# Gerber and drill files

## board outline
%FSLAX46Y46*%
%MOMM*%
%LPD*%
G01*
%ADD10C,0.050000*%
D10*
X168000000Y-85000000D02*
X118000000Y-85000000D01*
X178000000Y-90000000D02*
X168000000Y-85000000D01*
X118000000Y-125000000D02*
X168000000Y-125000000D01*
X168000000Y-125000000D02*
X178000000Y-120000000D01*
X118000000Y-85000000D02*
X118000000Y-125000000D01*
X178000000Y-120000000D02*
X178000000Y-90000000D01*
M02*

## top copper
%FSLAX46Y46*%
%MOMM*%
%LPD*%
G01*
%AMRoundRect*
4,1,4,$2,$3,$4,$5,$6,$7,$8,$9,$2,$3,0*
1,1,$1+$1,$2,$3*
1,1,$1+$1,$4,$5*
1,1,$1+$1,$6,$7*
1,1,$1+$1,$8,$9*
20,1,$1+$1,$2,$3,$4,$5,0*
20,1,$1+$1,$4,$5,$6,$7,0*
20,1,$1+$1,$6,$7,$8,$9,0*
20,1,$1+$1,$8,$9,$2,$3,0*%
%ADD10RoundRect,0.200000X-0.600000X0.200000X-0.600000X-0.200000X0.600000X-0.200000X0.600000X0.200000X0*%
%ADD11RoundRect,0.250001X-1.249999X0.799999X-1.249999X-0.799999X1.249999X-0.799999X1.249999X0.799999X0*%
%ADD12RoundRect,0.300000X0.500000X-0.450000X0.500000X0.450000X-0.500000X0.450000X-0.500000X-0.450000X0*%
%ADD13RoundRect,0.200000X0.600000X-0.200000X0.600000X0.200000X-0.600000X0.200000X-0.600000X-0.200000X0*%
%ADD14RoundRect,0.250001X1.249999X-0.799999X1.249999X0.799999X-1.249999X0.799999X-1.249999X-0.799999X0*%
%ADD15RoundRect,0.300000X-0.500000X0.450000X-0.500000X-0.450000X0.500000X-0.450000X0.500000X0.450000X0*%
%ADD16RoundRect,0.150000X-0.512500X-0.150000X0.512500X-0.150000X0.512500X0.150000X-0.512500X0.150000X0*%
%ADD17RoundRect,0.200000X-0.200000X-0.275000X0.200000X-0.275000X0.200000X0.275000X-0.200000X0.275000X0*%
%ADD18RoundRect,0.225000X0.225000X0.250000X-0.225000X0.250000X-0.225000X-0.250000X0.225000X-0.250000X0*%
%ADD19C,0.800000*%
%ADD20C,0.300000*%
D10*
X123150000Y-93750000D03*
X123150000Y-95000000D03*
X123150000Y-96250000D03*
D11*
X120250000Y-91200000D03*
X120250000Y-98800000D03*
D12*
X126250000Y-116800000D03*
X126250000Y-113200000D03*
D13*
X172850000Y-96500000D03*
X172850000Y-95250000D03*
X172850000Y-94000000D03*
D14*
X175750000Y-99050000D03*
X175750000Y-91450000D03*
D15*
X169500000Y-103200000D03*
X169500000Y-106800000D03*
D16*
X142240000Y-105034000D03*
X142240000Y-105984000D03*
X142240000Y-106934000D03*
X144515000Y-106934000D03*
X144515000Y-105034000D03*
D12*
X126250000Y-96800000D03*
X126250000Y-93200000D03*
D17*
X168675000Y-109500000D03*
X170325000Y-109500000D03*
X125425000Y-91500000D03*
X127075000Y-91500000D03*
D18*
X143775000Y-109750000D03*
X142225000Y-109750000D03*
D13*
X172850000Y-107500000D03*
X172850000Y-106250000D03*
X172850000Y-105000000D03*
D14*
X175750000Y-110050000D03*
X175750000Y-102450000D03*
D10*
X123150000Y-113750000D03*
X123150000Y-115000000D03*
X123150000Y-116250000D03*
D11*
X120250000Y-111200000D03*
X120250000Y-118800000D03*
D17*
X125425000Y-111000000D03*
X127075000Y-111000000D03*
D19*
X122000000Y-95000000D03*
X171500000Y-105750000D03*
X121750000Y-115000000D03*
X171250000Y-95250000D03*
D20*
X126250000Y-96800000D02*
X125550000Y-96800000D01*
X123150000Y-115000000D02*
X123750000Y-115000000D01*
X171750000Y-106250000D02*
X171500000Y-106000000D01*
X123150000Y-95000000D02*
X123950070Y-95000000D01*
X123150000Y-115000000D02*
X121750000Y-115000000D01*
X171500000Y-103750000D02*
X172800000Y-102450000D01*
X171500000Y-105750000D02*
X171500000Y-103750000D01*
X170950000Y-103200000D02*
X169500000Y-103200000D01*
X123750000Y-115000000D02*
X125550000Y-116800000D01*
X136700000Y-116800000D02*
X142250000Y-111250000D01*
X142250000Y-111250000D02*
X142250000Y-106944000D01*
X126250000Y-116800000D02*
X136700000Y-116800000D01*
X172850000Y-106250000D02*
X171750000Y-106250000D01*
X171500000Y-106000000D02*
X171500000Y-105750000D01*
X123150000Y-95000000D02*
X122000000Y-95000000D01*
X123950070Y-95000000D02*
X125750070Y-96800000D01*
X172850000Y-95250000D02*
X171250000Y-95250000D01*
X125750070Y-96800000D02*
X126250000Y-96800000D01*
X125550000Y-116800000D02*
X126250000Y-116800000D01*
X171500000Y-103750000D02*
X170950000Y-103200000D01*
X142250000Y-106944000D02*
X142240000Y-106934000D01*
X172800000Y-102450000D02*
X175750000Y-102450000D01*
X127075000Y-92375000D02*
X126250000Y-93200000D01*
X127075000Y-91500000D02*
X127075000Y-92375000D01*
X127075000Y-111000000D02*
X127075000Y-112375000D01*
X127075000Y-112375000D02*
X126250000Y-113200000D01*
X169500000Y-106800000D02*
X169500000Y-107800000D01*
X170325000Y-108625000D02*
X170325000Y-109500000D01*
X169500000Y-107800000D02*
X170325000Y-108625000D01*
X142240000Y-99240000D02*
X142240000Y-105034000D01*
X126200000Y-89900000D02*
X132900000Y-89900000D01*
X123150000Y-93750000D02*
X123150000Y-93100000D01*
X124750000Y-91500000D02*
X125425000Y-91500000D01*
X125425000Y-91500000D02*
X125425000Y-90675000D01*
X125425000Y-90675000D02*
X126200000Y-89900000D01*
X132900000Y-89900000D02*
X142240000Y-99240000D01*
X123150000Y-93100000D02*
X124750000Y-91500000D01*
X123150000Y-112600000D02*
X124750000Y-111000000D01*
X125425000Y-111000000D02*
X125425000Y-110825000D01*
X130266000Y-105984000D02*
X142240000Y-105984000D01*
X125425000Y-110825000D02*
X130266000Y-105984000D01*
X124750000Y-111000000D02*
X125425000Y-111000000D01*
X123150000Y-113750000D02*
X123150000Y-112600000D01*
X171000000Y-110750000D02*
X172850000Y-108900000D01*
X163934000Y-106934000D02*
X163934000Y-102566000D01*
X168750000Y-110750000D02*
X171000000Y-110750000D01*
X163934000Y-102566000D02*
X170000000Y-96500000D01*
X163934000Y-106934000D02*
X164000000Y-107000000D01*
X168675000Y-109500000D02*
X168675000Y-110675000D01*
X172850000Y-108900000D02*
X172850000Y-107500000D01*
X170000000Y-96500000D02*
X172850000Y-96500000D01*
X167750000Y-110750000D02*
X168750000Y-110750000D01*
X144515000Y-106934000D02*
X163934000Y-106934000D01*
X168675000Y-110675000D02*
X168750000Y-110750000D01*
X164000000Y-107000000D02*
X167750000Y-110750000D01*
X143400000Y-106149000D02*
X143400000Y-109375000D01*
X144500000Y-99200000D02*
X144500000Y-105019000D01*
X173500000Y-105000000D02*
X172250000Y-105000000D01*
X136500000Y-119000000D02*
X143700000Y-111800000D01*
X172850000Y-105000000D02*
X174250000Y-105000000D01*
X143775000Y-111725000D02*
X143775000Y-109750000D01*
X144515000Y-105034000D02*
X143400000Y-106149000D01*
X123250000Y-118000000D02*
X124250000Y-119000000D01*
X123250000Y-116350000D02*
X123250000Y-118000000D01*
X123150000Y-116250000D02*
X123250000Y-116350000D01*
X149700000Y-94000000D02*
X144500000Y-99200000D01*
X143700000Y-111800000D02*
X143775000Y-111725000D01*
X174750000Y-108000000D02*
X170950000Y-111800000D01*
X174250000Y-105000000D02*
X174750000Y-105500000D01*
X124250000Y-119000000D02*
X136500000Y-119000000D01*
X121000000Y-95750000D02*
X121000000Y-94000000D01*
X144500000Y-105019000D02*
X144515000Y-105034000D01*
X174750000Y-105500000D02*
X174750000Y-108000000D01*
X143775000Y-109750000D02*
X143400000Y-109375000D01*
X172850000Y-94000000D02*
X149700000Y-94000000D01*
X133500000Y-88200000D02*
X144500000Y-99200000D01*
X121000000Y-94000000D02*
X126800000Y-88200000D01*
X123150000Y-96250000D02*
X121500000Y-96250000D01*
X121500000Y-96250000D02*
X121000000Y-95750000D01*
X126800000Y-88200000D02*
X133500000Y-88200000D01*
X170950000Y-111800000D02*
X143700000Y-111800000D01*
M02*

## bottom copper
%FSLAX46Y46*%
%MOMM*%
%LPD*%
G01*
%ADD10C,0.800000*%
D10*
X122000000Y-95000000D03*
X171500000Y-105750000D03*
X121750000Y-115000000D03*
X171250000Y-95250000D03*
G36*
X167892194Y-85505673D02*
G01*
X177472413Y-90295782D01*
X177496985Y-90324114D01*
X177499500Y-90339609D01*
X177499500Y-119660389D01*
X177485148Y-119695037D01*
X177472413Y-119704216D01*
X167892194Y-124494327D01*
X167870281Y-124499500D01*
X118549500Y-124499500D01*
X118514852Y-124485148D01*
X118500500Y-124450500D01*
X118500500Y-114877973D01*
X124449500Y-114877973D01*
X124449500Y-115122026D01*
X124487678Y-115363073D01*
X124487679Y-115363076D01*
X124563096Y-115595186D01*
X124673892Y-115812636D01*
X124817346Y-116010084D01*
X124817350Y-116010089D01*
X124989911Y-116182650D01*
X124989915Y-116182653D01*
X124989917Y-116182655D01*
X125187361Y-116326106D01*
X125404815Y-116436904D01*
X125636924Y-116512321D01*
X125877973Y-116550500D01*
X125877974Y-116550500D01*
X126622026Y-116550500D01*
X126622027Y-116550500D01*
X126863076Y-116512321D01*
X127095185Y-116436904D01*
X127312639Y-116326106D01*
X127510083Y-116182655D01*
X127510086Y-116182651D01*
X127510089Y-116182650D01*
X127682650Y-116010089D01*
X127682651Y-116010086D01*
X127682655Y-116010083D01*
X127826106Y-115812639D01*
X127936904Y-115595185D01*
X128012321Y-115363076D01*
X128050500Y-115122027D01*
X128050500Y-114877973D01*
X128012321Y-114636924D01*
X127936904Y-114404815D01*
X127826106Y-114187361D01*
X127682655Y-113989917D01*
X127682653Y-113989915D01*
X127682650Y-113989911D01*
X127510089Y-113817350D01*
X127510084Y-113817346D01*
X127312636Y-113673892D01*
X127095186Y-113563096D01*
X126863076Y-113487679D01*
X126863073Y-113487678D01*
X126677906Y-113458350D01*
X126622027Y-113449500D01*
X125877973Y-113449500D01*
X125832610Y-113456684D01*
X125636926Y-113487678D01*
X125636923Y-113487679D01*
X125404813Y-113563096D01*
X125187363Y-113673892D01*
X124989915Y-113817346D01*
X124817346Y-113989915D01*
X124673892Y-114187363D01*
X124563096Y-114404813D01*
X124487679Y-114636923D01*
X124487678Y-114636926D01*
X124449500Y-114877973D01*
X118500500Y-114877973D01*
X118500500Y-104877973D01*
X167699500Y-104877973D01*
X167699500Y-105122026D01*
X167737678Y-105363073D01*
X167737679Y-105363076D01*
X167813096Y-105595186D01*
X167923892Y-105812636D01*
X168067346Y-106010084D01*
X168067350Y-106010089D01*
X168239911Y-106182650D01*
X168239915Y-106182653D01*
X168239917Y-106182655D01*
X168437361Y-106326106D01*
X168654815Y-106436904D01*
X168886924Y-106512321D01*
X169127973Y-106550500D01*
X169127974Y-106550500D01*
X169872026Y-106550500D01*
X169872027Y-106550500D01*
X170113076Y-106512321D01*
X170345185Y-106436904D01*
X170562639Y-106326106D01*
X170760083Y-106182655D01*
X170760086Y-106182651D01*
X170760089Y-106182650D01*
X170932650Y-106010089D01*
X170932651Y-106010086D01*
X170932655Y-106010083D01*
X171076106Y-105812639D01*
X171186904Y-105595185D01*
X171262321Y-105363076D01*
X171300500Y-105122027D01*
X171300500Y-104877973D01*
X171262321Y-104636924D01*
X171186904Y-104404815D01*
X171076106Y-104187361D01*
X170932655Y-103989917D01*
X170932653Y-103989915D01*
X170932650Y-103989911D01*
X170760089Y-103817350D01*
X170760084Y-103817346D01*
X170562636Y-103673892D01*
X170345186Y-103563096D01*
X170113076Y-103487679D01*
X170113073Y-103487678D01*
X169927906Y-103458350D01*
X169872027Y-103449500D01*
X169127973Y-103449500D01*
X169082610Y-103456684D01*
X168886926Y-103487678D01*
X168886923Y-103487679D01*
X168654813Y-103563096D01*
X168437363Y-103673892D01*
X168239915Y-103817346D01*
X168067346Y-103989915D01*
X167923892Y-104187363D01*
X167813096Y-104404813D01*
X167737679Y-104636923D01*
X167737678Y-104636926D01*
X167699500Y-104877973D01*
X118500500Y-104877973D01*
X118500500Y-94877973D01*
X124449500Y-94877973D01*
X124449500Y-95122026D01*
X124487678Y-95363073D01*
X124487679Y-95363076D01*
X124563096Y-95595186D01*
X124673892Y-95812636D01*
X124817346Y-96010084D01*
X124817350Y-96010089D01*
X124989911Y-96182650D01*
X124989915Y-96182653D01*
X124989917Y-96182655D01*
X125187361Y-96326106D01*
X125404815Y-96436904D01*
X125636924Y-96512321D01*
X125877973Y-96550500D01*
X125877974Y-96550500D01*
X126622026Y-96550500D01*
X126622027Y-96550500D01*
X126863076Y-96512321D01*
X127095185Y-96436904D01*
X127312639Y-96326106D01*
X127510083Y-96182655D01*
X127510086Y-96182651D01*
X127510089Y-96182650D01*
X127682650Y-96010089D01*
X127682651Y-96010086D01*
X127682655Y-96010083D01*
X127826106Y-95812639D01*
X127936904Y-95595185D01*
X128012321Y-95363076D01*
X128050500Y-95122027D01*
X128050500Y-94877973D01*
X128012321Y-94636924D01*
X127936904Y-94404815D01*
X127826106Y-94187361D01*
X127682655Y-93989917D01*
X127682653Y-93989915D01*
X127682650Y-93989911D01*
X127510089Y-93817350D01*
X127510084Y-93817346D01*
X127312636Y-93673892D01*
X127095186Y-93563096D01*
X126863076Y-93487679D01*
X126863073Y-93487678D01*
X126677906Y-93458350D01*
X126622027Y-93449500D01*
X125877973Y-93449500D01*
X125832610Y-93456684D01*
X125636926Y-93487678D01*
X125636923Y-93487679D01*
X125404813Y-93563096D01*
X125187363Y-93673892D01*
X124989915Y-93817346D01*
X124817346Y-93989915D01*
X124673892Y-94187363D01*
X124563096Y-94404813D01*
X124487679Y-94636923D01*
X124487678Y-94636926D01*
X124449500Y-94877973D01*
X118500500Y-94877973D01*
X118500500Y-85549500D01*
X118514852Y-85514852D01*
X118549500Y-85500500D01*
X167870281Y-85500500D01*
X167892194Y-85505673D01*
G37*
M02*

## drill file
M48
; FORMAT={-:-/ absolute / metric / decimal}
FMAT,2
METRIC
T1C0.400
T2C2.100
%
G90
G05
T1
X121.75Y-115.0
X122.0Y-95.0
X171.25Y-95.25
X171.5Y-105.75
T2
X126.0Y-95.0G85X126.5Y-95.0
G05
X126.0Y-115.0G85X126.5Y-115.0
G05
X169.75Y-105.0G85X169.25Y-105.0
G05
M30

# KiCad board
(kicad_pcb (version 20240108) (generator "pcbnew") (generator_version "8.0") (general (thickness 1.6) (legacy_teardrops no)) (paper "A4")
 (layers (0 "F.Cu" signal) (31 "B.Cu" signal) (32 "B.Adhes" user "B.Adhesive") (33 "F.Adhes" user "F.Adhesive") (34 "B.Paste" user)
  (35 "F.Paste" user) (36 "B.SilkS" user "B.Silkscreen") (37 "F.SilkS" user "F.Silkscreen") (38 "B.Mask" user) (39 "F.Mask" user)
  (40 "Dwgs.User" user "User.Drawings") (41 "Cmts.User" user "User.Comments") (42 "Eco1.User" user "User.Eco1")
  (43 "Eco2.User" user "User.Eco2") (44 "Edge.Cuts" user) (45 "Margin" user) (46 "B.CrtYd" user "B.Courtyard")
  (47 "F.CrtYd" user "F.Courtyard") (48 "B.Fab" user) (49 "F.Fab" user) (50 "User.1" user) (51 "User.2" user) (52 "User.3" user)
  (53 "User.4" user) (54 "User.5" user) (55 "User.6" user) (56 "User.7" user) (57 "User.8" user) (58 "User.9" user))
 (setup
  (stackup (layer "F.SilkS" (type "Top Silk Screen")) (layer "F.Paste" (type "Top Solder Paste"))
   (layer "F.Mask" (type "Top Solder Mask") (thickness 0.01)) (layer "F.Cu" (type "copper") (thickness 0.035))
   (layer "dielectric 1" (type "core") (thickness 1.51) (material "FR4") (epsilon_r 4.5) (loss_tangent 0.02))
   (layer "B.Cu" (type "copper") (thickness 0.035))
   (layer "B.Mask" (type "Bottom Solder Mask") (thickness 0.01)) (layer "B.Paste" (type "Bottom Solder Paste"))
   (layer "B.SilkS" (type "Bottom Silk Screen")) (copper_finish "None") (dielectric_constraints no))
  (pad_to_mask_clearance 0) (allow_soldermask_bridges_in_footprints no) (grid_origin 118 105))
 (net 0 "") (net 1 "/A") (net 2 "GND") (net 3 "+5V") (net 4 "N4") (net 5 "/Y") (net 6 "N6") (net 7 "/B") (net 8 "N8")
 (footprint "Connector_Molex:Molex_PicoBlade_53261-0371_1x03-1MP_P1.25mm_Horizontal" (layer "F.Cu") (at 120.75 95 -90)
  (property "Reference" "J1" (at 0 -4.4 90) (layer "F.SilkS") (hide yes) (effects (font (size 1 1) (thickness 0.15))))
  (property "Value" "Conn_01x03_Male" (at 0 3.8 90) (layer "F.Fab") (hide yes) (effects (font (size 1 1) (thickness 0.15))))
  (pad "1" smd roundrect (at -1.25 -2.4 270) (size 0.8 1.6) (layers "F.Cu" "F.Paste" "F.Mask") (roundrect_rratio 0.25) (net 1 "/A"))
  (pad "2" smd roundrect (at 0 -2.4 270) (size 0.8 1.6) (layers "F.Cu" "F.Paste" "F.Mask") (roundrect_rratio 0.25) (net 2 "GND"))
  (pad "3" smd roundrect (at 1.25 -2.4 270) (size 0.8 1.6) (layers "F.Cu" "F.Paste" "F.Mask") (roundrect_rratio 0.25) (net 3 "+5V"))
  (pad "MP" smd roundrect (at -3.8 0.5 270) (size 2.1 3) (layers "F.Cu" "F.Paste" "F.Mask") (roundrect_rratio 0.1190480952))
  (pad "MP" smd roundrect (at 3.8 0.5 270) (size 2.1 3) (layers "F.Cu" "F.Paste" "F.Mask") (roundrect_rratio 0.1190480952)))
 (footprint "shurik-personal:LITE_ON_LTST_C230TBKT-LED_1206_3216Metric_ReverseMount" (layer "F.Cu") (at 126.25 115 90)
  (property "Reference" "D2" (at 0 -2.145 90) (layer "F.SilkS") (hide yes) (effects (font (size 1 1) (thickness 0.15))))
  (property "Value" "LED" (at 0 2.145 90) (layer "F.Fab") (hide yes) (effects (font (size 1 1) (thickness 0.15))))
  (pad "" np_thru_hole oval (at 0 0 90) (size 2.1 2.6) (drill oval 2.1 2.6) (layers "F&B.Cu" "*.Mask"))
  (pad "1" smd roundrect (at -1.8 0 90) (size 1.5 1.6) (layers "F.Cu" "F.Paste" "F.Mask") (roundrect_rratio 0.2) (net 2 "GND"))
  (pad "2" smd roundrect (at 1.8 0 90) (size 1.5 1.6) (layers "F.Cu" "F.Paste" "F.Mask") (roundrect_rratio 0.2) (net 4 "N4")))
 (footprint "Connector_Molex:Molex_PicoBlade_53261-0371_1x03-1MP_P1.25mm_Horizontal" (layer "F.Cu") (at 175.25 95.25 90)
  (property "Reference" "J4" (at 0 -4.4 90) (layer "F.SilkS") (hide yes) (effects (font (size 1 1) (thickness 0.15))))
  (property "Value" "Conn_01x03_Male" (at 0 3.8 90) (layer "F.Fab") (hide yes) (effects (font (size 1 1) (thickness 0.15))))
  (pad "1" smd roundrect (at -1.25 -2.4 90) (size 0.8 1.6) (layers "F.Cu" "F.Paste" "F.Mask") (roundrect_rratio 0.25) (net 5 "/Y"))
  (pad "2" smd roundrect (at 0 -2.4 90) (size 0.8 1.6) (layers "F.Cu" "F.Paste" "F.Mask") (roundrect_rratio 0.25) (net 2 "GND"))
  (pad "3" smd roundrect (at 1.25 -2.4 90) (size 0.8 1.6) (layers "F.Cu" "F.Paste" "F.Mask") (roundrect_rratio 0.25) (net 3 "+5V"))
  (pad "MP" smd roundrect (at -3.8 0.5 90) (size 2.1 3) (layers "F.Cu" "F.Paste" "F.Mask") (roundrect_rratio 0.1190480952))
  (pad "MP" smd roundrect (at 3.8 0.5 90) (size 2.1 3) (layers "F.Cu" "F.Paste" "F.Mask") (roundrect_rratio 0.1190480952)))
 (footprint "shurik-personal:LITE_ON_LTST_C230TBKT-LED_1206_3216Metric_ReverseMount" (layer "F.Cu") (at 169.5 105 -90)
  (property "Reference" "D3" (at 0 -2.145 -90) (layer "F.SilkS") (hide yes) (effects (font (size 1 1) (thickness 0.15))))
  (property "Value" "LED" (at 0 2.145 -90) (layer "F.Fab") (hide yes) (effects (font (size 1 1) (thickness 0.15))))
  (pad "" np_thru_hole oval (at 0 0 270) (size 2.1 2.6) (drill oval 2.1 2.6) (layers "F&B.Cu" "*.Mask"))
  (pad "1" smd roundrect (at -1.8 0 270) (size 1.5 1.6) (layers "F.Cu" "F.Paste" "F.Mask") (roundrect_rratio 0.2) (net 2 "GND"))
  (pad "2" smd roundrect (at 1.8 0 270) (size 1.5 1.6) (layers "F.Cu" "F.Paste" "F.Mask") (roundrect_rratio 0.2) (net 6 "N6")))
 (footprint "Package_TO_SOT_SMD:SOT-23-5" (layer "F.Cu") (at 143.3775 105.984)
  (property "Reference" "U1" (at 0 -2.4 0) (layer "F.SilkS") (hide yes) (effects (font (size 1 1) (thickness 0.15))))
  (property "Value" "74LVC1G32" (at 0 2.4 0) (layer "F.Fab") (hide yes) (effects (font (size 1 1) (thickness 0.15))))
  (pad "1" smd roundrect (at -1.1375 -0.95) (size 1.325 0.6) (layers "F.Cu" "F.Paste" "F.Mask") (roundrect_rratio 0.25) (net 1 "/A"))
  (pad "2" smd roundrect (at -1.1375 0) (size 1.325 0.6) (layers "F.Cu" "F.Paste" "F.Mask") (roundrect_rratio 0.25) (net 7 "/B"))
  (pad "3" smd roundrect (at -1.1375 0.95) (size 1.325 0.6) (layers "F.Cu" "F.Paste" "F.Mask") (roundrect_rratio 0.25) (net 2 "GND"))
  (pad "4" smd roundrect (at 1.1375 0.95) (size 1.325 0.6) (layers "F.Cu" "F.Paste" "F.Mask") (roundrect_rratio 0.25) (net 5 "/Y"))
  (pad "5" smd roundrect (at 1.1375 -0.95) (size 1.325 0.6) (layers "F.Cu" "F.Paste" "F.Mask") (roundrect_rratio 0.25) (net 3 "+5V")))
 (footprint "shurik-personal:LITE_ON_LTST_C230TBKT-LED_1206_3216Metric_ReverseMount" (layer "F.Cu") (at 126.25 95 90)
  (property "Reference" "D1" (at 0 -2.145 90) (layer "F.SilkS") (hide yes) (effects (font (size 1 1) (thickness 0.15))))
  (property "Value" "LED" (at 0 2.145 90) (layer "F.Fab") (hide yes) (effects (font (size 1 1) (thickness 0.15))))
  (pad "" np_thru_hole oval (at 0 0 90) (size 2.1 2.6) (drill oval 2.1 2.6) (layers "F&B.Cu" "*.Mask"))
  (pad "1" smd roundrect (at -1.8 0 90) (size 1.5 1.6) (layers "F.Cu" "F.Paste" "F.Mask") (roundrect_rratio 0.2) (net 2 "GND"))
  (pad "2" smd roundrect (at 1.8 0 90) (size 1.5 1.6) (layers "F.Cu" "F.Paste" "F.Mask") (roundrect_rratio 0.2) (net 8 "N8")))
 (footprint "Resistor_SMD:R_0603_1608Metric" (layer "F.Cu") (at 169.5 109.5)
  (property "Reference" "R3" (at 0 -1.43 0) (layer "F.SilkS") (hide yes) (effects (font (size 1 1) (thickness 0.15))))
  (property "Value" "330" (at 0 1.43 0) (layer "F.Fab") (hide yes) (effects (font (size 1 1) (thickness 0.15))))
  (pad "1" smd roundrect (at -0.825 0) (size 0.8 0.95) (layers "F.Cu" "F.Paste" "F.Mask") (roundrect_rratio 0.25) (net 5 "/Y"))
  (pad "2" smd roundrect (at 0.825 0) (size 0.8 0.95) (layers "F.Cu" "F.Paste" "F.Mask") (roundrect_rratio 0.25) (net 6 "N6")))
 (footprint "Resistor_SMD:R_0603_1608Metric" (layer "F.Cu") (at 126.25 91.5)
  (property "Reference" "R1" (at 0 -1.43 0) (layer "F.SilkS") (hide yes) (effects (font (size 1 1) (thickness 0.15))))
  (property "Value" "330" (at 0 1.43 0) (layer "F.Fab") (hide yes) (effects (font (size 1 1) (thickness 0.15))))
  (pad "1" smd roundrect (at -0.825 0) (size 0.8 0.95) (layers "F.Cu" "F.Paste" "F.Mask") (roundrect_rratio 0.25) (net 1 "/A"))
  (pad "2" smd roundrect (at 0.825 0) (size 0.8 0.95) (layers "F.Cu" "F.Paste" "F.Mask") (roundrect_rratio 0.25) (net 8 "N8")))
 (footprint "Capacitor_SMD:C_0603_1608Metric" (layer "F.Cu") (at 143 109.75 180)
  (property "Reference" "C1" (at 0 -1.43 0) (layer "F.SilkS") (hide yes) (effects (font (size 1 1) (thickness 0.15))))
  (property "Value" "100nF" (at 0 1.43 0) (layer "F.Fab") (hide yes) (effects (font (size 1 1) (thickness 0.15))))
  (pad "1" smd roundrect (at -0.775 0 180) (size 0.9 0.95) (layers "F.Cu" "F.Paste" "F.Mask") (roundrect_rratio 0.25) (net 3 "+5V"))
  (pad "2" smd roundrect (at 0.775 0 180) (size 0.9 0.95) (layers "F.Cu" "F.Paste" "F.Mask") (roundrect_rratio 0.25) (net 2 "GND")))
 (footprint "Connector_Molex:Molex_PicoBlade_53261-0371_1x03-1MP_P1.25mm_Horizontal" (layer "F.Cu") (at 175.25 106.25 90)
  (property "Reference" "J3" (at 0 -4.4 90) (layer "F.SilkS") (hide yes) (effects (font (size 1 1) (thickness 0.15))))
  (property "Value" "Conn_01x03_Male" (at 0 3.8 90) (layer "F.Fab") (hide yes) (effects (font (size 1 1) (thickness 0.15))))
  (pad "1" smd roundrect (at -1.25 -2.4 90) (size 0.8 1.6) (layers "F.Cu" "F.Paste" "F.Mask") (roundrect_rratio 0.25) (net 5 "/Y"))
  (pad "2" smd roundrect (at 0 -2.4 90) (size 0.8 1.6) (layers "F.Cu" "F.Paste" "F.Mask") (roundrect_rratio 0.25) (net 2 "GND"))
  (pad "3" smd roundrect (at 1.25 -2.4 90) (size 0.8 1.6) (layers "F.Cu" "F.Paste" "F.Mask") (roundrect_rratio 0.25) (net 3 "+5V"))
  (pad "MP" smd roundrect (at -3.8 0.5 90) (size 2.1 3) (layers "F.Cu" "F.Paste" "F.Mask") (roundrect_rratio 0.1190480952))
  (pad "MP" smd roundrect (at 3.8 0.5 90) (size 2.1 3) (layers "F.Cu" "F.Paste" "F.Mask") (roundrect_rratio 0.1190480952)))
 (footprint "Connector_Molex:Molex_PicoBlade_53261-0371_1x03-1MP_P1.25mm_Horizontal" (layer "F.Cu") (at 120.75 115 -90)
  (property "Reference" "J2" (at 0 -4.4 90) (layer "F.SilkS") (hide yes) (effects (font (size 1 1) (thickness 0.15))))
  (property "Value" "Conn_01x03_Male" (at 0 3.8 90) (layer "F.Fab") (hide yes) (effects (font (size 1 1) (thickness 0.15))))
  (pad "1" smd roundrect (at -1.25 -2.4 270) (size 0.8 1.6) (layers "F.Cu" "F.Paste" "F.Mask") (roundrect_rratio 0.25) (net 7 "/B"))
  (pad "2" smd roundrect (at 0 -2.4 270) (size 0.8 1.6) (layers "F.Cu" "F.Paste" "F.Mask") (roundrect_rratio 0.25) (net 2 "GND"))
  (pad "3" smd roundrect (at 1.25 -2.4 270) (size 0.8 1.6) (layers "F.Cu" "F.Paste" "F.Mask") (roundrect_rratio 0.25) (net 3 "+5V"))
  (pad "MP" smd roundrect (at -3.8 0.5 270) (size 2.1 3) (layers "F.Cu" "F.Paste" "F.Mask") (roundrect_rratio 0.1190480952))
  (pad "MP" smd roundrect (at 3.8 0.5 270) (size 2.1 3) (layers "F.Cu" "F.Paste" "F.Mask") (roundrect_rratio 0.1190480952)))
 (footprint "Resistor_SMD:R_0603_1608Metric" (layer "F.Cu") (at 126.25 111)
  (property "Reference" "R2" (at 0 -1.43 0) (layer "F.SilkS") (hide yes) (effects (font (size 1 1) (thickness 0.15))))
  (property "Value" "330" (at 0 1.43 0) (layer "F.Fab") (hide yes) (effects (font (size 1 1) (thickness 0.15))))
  (pad "1" smd roundrect (at -0.825 0) (size 0.8 0.95) (layers "F.Cu" "F.Paste" "F.Mask") (roundrect_rratio 0.25) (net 7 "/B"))
  (pad "2" smd roundrect (at 0.825 0) (size 0.8 0.95) (layers "F.Cu" "F.Paste" "F.Mask") (roundrect_rratio 0.25) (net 4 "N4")))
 (gr_line (start 168 85) (end 118 85) (stroke (width 0.05) (type solid)) (layer "Edge.Cuts"))
 (gr_line (start 178 90) (end 168 85) (stroke (width 0.05) (type solid)) (layer "Edge.Cuts"))
 (gr_line (start 118 125) (end 168 125) (stroke (width 0.05) (type solid)) (layer "Edge.Cuts"))
 (gr_line (start 168 125) (end 178 120) (stroke (width 0.05) (type solid)) (layer "Edge.Cuts"))
 (gr_line (start 118 85) (end 118 125) (stroke (width 0.05) (type solid)) (layer "Edge.Cuts"))
 (gr_line (start 178 120) (end 178 90) (stroke (width 0.05) (type solid)) (layer "Edge.Cuts"))
 (segment (start 126.25 96.8) (end 125.55 96.8) (width 0.3) (layer "F.Cu") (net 2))
 (segment (start 123.15 115) (end 123.75 115) (width 0.3) (layer "F.Cu") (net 2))
 (segment (start 171.75 106.25) (end 171.5 106) (width 0.3) (layer "F.Cu") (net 2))
 (segment (start 123.15 95) (end 123.95007 95) (width 0.3) (layer "F.Cu") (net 2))
 (segment (start 123.15 115) (end 121.75 115) (width 0.3) (layer "F.Cu") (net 2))
 (segment (start 171.5 103.75) (end 172.8 102.45) (width 0.3) (layer "F.Cu") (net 2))
 (segment (start 171.5 105.75) (end 171.5 103.75) (width 0.3) (layer "F.Cu") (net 2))
 (segment (start 170.95 103.2) (end 169.5 103.2) (width 0.3) (layer "F.Cu") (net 2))
 (segment (start 123.75 115) (end 125.55 116.8) (width 0.3) (layer "F.Cu") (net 2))
 (segment (start 136.7 116.8) (end 142.25 111.25) (width 0.3) (layer "F.Cu") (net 2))
 (segment (start 142.25 111.25) (end 142.25 106.944) (width 0.3) (layer "F.Cu") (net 2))
 (segment (start 126.25 116.8) (end 136.7 116.8) (width 0.3) (layer "F.Cu") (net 2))
 (segment (start 172.85 106.25) (end 171.75 106.25) (width 0.3) (layer "F.Cu") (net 2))
 (segment (start 171.5 106) (end 171.5 105.75) (width 0.3) (layer "F.Cu") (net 2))
 (segment (start 123.15 95) (end 122 95) (width 0.3) (layer "F.Cu") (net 2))
 (segment (start 123.95007 95) (end 125.75007 96.8) (width 0.3) (layer "F.Cu") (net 2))
 (segment (start 172.85 95.25) (end 171.25 95.25) (width 0.3) (layer "F.Cu") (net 2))
 (segment (start 125.75007 96.8) (end 126.25 96.8) (width 0.3) (layer "F.Cu") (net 2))
 (segment (start 125.55 116.8) (end 126.25 116.8) (width 0.3) (layer "F.Cu") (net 2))
 (segment (start 171.5 103.75) (end 170.95 103.2) (width 0.3) (layer "F.Cu") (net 2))
 (segment (start 142.25 106.944) (end 142.24 106.934) (width 0.3) (layer "F.Cu") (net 2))
 (segment (start 172.8 102.45) (end 175.75 102.45) (width 0.3) (layer "F.Cu") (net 2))
 (via (at 122 95) (size 0.8) (drill 0.4) (layers "F.Cu" "B.Cu") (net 2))
 (via (at 171.5 105.75) (size 0.8) (drill 0.4) (layers "F.Cu" "B.Cu") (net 2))
 (via (at 121.75 115) (size 0.8) (drill 0.4) (layers "F.Cu" "B.Cu") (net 2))
 (via (at 171.25 95.25) (size 0.8) (drill 0.4) (layers "F.Cu" "B.Cu") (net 2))
 (segment (start 127.075 92.375) (end 126.25 93.2) (width 0.3) (layer "F.Cu") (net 8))
 (segment (start 127.075 91.5) (end 127.075 92.375) (width 0.3) (layer "F.Cu") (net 8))
 (segment (start 127.075 111) (end 127.075 112.375) (width 0.3) (layer "F.Cu") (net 4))
 (segment (start 127.075 112.375) (end 126.25 113.2) (width 0.3) (layer "F.Cu") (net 4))
 (segment (start 169.5 106.8) (end 169.5 107.8) (width 0.3) (layer "F.Cu") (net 6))
 (segment (start 170.325 108.625) (end 170.325 109.5) (width 0.3) (layer "F.Cu") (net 6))
 (segment (start 169.5 107.8) (end 170.325 108.625) (width 0.3) (layer "F.Cu") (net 6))
 (segment (start 142.24 99.24) (end 142.24 105.034) (width 0.3) (layer "F.Cu") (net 1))
 (segment (start 126.2 89.9) (end 132.9 89.9) (width 0.3) (layer "F.Cu") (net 1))
 (segment (start 123.15 93.75) (end 123.15 93.1) (width 0.3) (layer "F.Cu") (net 1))
 (segment (start 124.75 91.5) (end 125.425 91.5) (width 0.3) (layer "F.Cu") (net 1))
 (segment (start 125.425 91.5) (end 125.425 90.675) (width 0.3) (layer "F.Cu") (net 1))
 (segment (start 125.425 90.675) (end 126.2 89.9) (width 0.3) (layer "F.Cu") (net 1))
 (segment (start 132.9 89.9) (end 142.24 99.24) (width 0.3) (layer "F.Cu") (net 1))
 (segment (start 123.15 93.1) (end 124.75 91.5) (width 0.3) (layer "F.Cu") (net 1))
 (segment (start 123.15 112.6) (end 124.75 111) (width 0.3) (layer "F.Cu") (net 7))
 (segment (start 125.425 111) (end 125.425 110.825) (width 0.3) (layer "F.Cu") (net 7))
 (segment (start 130.266 105.984) (end 142.24 105.984) (width 0.3) (layer "F.Cu") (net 7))
 (segment (start 125.425 110.825) (end 130.266 105.984) (width 0.3) (layer "F.Cu") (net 7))
 (segment (start 124.75 111) (end 125.425 111) (width 0.3) (layer "F.Cu") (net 7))
 (segment (start 123.15 113.75) (end 123.15 112.6) (width 0.3) (layer "F.Cu") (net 7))
 (segment (start 171 110.75) (end 172.85 108.9) (width 0.3) (layer "F.Cu") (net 5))
 (segment (start 163.934 106.934) (end 163.934 102.566) (width 0.3) (layer "F.Cu") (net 5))
 (segment (start 168.75 110.75) (end 171 110.75) (width 0.3) (layer "F.Cu") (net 5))
 (segment (start 163.934 102.566) (end 170 96.5) (width 0.3) (layer "F.Cu") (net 5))
 (segment (start 163.934 106.934) (end 164 107) (width 0.3) (layer "F.Cu") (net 5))
 (segment (start 168.675 109.5) (end 168.675 110.675) (width 0.3) (layer "F.Cu") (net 5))
 (segment (start 172.85 108.9) (end 172.85 107.5) (width 0.3) (layer "F.Cu") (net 5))
 (segment (start 170 96.5) (end 172.85 96.5) (width 0.3) (layer "F.Cu") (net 5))
 (segment (start 167.75 110.75) (end 168.75 110.75) (width 0.3) (layer "F.Cu") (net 5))
 (segment (start 144.515 106.934) (end 163.934 106.934) (width 0.3) (layer "F.Cu") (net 5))
 (segment (start 168.675 110.675) (end 168.75 110.75) (width 0.3) (layer "F.Cu") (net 5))
 (segment (start 164 107) (end 167.75 110.75) (width 0.3) (layer "F.Cu") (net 5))
 (segment (start 143.4 106.149) (end 143.4 109.375) (width 0.3) (layer "F.Cu") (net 3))
 (segment (start 144.5 99.2) (end 144.5 105.019) (width 0.3) (layer "F.Cu") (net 3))
 (segment (start 173.5 105) (end 172.25 105) (width 0.3) (layer "F.Cu") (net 3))
 (segment (start 136.5 119) (end 143.7 111.8) (width 0.3) (layer "F.Cu") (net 3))
 (segment (start 172.85 105) (end 174.25 105) (width 0.3) (layer "F.Cu") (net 3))
 (segment (start 143.775 111.725) (end 143.775 109.75) (width 0.3) (layer "F.Cu") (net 3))
 (segment (start 144.515 105.034) (end 143.4 106.149) (width 0.3) (layer "F.Cu") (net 3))
 (segment (start 123.25 118) (end 124.25 119) (width 0.3) (layer "F.Cu") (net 3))
 (segment (start 123.25 116.35) (end 123.25 118) (width 0.3) (layer "F.Cu") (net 3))
 (segment (start 123.15 116.25) (end 123.25 116.35) (width 0.3) (layer "F.Cu") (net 3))
 (segment (start 149.7 94) (end 144.5 99.2) (width 0.3) (layer "F.Cu") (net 3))
 (segment (start 143.7 111.8) (end 143.775 111.725) (width 0.3) (layer "F.Cu") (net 3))
 (segment (start 174.75 108) (end 170.95 111.8) (width 0.3) (layer "F.Cu") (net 3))
 (segment (start 174.25 105) (end 174.75 105.5) (width 0.3) (layer "F.Cu") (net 3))
 (segment (start 124.25 119) (end 136.5 119) (width 0.3) (layer "F.Cu") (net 3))
 (segment (start 121 95.75) (end 121 94) (width 0.3) (layer "F.Cu") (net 3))
 (segment (start 144.5 105.019) (end 144.515 105.034) (width 0.3) (layer "F.Cu") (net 3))
 (segment (start 174.75 105.5) (end 174.75 108) (width 0.3) (layer "F.Cu") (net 3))
 (segment (start 143.775 109.75) (end 143.4 109.375) (width 0.3) (layer "F.Cu") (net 3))
 (segment (start 172.85 94) (end 149.7 94) (width 0.3) (layer "F.Cu") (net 3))
 (segment (start 133.5 88.2) (end 144.5 99.2) (width 0.3) (layer "F.Cu") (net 3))
 (segment (start 121 94) (end 126.8 88.2) (width 0.3) (layer "F.Cu") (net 3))
 (segment (start 123.15 96.25) (end 121.5 96.25) (width 0.3) (layer "F.Cu") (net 3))
 (segment (start 121.5 96.25) (end 121 95.75) (width 0.3) (layer "F.Cu") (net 3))
 (segment (start 126.8 88.2) (end 133.5 88.2) (width 0.3) (layer "F.Cu") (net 3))
 (segment (start 170.95 111.8) (end 143.7 111.8) (width 0.3) (layer "F.Cu") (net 3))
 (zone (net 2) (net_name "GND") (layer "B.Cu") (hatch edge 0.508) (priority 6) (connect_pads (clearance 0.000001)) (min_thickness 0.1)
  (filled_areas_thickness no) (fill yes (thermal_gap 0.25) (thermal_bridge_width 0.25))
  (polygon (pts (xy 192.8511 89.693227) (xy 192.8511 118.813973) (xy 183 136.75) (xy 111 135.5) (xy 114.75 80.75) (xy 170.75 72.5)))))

